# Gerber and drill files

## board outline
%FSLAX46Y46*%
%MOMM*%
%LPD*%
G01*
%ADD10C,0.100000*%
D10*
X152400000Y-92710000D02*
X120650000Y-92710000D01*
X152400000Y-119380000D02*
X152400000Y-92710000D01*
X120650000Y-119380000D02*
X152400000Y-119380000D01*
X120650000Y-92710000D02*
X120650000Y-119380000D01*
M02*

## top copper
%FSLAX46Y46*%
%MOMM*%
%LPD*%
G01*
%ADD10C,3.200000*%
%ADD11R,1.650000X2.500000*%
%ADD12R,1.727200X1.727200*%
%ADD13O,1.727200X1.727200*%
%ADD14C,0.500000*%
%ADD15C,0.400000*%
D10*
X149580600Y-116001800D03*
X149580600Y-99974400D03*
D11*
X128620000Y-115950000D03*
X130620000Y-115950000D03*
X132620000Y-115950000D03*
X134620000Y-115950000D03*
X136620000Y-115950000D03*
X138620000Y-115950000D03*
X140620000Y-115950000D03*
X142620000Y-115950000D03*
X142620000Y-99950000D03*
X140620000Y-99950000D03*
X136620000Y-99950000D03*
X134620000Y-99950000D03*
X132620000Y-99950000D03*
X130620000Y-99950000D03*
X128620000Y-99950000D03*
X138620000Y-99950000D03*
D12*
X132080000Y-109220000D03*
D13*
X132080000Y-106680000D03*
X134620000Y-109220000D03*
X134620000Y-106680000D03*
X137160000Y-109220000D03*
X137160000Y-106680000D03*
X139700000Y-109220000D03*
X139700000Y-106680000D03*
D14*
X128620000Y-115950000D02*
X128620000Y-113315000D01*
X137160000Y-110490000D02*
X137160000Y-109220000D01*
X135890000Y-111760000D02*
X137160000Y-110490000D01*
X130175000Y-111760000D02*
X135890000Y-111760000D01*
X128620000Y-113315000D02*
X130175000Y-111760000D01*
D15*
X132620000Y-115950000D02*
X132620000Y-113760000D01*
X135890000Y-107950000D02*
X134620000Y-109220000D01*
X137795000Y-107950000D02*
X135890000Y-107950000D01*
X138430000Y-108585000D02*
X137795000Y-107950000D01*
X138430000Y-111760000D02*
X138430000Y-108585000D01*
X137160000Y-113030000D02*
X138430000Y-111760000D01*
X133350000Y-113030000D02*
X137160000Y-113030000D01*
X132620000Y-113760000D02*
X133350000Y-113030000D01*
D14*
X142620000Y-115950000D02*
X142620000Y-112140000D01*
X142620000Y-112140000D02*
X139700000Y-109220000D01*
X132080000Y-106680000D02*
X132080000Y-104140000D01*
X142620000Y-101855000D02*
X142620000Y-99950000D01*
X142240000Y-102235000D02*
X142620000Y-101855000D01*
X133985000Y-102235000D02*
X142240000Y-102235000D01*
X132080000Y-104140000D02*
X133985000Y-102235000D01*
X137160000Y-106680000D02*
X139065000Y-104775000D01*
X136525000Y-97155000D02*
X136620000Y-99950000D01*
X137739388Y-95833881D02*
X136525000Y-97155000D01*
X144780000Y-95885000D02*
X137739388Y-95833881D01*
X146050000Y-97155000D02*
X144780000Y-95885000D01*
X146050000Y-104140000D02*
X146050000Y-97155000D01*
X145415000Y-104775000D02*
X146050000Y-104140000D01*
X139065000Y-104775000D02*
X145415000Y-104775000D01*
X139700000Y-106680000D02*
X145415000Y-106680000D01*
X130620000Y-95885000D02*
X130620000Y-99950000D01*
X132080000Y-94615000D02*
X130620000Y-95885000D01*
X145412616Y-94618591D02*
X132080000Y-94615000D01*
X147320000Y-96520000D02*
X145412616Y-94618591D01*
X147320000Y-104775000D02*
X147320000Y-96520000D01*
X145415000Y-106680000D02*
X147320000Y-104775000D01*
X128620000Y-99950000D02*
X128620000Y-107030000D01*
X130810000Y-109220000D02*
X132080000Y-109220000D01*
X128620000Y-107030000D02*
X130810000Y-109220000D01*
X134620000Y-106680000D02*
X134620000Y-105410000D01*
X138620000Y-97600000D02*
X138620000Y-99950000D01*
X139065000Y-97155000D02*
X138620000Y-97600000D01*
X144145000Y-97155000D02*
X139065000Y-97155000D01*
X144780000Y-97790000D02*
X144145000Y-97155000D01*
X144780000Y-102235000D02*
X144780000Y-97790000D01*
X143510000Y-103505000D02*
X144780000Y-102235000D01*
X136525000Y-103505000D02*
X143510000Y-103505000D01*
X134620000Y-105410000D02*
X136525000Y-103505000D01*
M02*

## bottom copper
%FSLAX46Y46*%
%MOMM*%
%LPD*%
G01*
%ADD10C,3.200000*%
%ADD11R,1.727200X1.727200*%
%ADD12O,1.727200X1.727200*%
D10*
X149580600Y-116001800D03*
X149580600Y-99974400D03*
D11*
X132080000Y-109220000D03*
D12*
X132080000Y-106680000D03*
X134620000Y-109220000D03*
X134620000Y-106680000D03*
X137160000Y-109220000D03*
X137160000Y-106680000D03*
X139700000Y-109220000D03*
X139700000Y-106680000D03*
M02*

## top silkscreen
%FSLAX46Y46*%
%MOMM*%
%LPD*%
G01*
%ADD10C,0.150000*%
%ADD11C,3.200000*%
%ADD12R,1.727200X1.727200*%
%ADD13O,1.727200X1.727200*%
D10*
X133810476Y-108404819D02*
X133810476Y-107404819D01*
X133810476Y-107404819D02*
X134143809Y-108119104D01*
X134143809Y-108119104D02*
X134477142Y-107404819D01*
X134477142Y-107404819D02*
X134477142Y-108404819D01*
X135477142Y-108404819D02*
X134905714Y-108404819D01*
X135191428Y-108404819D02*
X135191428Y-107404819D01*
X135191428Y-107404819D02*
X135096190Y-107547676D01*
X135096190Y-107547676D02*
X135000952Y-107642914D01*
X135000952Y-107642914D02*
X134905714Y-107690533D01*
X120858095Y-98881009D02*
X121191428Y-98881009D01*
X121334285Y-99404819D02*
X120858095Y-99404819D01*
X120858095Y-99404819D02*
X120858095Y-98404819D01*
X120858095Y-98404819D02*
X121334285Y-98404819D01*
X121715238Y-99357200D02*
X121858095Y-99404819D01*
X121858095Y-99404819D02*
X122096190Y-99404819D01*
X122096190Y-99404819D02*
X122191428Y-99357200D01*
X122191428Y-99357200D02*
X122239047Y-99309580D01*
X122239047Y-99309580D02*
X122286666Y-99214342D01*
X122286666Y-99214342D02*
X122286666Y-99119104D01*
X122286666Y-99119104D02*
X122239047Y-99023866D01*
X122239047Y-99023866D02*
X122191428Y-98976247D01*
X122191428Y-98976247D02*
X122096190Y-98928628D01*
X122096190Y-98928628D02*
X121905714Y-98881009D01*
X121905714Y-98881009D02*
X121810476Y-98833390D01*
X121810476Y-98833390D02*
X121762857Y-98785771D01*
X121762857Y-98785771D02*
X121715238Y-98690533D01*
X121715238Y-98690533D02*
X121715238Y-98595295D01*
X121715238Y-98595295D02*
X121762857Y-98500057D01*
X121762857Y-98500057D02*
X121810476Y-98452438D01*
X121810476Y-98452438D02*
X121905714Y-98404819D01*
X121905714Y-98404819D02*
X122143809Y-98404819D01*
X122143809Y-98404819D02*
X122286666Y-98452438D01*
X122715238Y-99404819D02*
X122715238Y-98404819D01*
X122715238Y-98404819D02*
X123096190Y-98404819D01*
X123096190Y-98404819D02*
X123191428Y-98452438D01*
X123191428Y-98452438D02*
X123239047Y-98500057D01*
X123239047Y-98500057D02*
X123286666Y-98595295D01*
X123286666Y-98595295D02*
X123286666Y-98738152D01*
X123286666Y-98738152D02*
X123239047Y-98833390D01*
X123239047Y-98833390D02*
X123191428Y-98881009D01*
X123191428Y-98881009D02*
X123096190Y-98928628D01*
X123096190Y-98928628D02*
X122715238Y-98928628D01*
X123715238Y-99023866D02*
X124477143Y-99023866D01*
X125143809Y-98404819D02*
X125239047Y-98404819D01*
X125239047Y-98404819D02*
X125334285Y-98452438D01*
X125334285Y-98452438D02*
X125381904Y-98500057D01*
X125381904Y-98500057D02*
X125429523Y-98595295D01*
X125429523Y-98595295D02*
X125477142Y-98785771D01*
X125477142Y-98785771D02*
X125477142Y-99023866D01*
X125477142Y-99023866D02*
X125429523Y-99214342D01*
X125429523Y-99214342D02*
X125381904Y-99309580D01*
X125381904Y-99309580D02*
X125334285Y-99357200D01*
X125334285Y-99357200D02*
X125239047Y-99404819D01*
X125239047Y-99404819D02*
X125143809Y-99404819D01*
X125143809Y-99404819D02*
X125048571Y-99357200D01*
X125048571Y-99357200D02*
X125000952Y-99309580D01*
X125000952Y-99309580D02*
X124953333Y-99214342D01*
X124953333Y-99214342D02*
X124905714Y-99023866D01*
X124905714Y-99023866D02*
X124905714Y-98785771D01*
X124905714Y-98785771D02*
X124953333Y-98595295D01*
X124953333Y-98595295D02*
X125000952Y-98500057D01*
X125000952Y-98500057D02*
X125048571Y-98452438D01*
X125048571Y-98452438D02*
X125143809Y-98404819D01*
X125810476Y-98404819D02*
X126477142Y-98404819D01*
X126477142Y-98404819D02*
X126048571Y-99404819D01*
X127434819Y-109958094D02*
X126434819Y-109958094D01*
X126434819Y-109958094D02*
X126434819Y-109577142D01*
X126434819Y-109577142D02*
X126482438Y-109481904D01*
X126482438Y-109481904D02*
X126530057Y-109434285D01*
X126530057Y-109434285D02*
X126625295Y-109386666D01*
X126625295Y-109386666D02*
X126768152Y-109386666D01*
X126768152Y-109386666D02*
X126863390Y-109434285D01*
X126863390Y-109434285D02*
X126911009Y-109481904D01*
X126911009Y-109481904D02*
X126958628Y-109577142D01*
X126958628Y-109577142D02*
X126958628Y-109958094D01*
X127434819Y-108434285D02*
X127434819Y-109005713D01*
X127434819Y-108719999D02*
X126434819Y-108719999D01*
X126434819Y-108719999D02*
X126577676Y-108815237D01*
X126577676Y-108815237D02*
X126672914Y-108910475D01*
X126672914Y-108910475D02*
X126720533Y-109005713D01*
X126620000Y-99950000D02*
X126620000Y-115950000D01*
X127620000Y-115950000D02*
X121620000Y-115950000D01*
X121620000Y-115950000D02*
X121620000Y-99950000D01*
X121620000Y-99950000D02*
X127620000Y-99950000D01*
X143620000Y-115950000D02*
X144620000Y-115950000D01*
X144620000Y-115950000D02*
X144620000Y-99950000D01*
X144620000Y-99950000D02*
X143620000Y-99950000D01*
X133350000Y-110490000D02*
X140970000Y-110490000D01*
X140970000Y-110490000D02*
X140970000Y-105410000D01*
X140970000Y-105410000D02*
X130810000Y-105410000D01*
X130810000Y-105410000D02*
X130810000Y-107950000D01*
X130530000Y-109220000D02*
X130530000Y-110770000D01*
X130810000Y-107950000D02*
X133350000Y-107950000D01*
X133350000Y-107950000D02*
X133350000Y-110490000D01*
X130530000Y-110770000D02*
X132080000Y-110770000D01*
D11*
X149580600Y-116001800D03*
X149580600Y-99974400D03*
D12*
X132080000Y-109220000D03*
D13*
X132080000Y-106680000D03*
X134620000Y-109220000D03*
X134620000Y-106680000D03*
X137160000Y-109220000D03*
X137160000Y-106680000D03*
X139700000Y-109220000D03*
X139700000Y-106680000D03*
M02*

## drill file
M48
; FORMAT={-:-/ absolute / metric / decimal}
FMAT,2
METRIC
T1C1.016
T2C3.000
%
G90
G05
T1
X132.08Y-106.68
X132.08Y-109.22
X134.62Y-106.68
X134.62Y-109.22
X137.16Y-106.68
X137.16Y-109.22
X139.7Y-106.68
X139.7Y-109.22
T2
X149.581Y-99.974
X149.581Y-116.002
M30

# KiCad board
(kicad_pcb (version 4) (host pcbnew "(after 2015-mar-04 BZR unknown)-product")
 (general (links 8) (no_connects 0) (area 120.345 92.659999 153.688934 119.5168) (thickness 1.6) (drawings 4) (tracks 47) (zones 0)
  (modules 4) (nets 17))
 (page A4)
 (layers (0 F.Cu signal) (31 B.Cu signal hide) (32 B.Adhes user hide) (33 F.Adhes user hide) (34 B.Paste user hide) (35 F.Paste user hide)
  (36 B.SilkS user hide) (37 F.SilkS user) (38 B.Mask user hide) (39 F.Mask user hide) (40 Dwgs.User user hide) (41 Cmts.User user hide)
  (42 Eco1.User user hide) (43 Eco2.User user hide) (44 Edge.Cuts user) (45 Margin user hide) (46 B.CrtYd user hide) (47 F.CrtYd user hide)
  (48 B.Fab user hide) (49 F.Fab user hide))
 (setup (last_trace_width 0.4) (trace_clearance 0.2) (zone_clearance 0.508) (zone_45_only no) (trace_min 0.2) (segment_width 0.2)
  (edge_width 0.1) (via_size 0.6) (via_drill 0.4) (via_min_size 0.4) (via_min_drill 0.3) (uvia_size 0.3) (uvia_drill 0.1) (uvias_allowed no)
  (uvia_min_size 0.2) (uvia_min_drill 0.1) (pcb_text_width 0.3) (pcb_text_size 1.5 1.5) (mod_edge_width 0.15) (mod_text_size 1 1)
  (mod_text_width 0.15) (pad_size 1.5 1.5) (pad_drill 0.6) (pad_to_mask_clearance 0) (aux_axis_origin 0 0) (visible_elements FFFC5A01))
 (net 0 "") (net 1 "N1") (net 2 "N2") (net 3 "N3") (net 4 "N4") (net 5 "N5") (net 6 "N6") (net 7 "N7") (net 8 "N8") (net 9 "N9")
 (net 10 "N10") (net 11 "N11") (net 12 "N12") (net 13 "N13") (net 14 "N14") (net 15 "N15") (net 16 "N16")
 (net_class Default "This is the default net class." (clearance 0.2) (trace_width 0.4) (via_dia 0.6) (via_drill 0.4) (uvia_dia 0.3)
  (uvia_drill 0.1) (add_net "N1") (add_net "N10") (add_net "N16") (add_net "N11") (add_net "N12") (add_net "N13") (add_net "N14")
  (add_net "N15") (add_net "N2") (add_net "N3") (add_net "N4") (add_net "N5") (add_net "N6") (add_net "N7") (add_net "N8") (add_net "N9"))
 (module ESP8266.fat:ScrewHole (layer F.Cu) (at 149.5806 116.0018)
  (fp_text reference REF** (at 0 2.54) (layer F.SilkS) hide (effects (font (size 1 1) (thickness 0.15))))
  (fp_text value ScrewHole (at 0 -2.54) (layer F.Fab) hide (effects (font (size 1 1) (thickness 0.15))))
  (pad 1 thru_hole circle (at 0 0) (size 3.2 3.2) (drill 3) (layers *.Cu *.Mask F.SilkS)))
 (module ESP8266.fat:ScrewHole (layer F.Cu) (at 149.5806 99.9744)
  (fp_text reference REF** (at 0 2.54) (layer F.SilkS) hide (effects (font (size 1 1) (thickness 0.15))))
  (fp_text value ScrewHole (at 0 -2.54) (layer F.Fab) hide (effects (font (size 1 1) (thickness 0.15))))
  (pad 1 thru_hole circle (at 0 0) (size 3.2 3.2) (drill 3) (layers *.Cu *.Mask F.SilkS)))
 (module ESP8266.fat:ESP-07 (layer F.Cu) (at 134.62 107.95)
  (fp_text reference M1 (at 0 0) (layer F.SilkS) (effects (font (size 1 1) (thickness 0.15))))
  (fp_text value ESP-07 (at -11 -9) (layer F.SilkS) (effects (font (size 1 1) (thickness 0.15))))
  (fp_line (start -8 -8) (end -8 8) (layer F.SilkS) (width 0.15))
  (fp_line (start -7 8) (end -13 8) (layer F.SilkS) (width 0.15))
  (fp_line (start -13 8) (end -13 -8) (layer F.SilkS) (width 0.15))
  (fp_line (start -13 -8) (end -7 -8) (layer F.SilkS) (width 0.15))
  (fp_line (start 9 8) (end 10 8) (layer F.SilkS) (width 0.15))
  (fp_line (start 10 8) (end 10 -8) (layer F.SilkS) (width 0.15))
  (fp_line (start 10 -8) (end 9 -8) (layer F.SilkS) (width 0.15))
  (pad 1 smd rect (at -6 8) (size 1.65 2.5) (layers F.Cu F.Paste F.Mask) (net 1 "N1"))
  (pad 2 smd rect (at -4 8) (size 1.65 2.5) (layers F.Cu F.Paste F.Mask) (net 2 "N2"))
  (pad 3 smd rect (at -2 8) (size 1.65 2.5) (layers F.Cu F.Paste F.Mask) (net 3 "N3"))
  (pad 4 smd rect (at 0 8) (size 1.65 2.5) (layers F.Cu F.Paste F.Mask) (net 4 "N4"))
  (pad 5 smd rect (at 2 8) (size 1.65 2.5) (layers F.Cu F.Paste F.Mask) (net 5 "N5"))
  (pad 6 smd rect (at 4 8) (size 1.65 2.5) (layers F.Cu F.Paste F.Mask) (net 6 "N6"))
  (pad 7 smd rect (at 6 8) (size 1.65 2.5) (layers F.Cu F.Paste F.Mask) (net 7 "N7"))
  (pad 8 smd rect (at 8 8) (size 1.65 2.5) (layers F.Cu F.Paste F.Mask) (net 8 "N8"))
  (pad 9 smd rect (at 8 -8) (size 1.65 2.5) (layers F.Cu F.Paste F.Mask) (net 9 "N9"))
  (pad 10 smd rect (at 6 -8) (size 1.65 2.5) (layers F.Cu F.Paste F.Mask) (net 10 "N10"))
  (pad 12 smd rect (at 2 -8) (size 1.65 2.5) (layers F.Cu F.Paste F.Mask) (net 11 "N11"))
  (pad 13 smd rect (at 0 -8) (size 1.65 2.5) (layers F.Cu F.Paste F.Mask) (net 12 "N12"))
  (pad 14 smd rect (at -2 -8) (size 1.65 2.5) (layers F.Cu F.Paste F.Mask) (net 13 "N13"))
  (pad 15 smd rect (at -4 -8) (size 1.65 2.5) (layers F.Cu F.Paste F.Mask) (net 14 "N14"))
  (pad 16 smd rect (at -6 -8) (size 1.65 2.5) (layers F.Cu F.Paste F.Mask) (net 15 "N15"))
  (pad 11 smd rect (at 4 -8) (size 1.65 2.5) (layers F.Cu F.Paste F.Mask) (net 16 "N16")))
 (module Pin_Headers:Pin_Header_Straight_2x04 (layer F.Cu) (at 132.08 109.22 90)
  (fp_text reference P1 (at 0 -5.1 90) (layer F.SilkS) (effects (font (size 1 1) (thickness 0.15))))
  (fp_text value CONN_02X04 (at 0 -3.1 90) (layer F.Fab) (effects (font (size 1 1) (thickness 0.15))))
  (fp_line (start -1.27 1.27) (end -1.27 8.89) (layer F.SilkS) (width 0.15))
  (fp_line (start -1.27 8.89) (end 3.81 8.89) (layer F.SilkS) (width 0.15))
  (fp_line (start 3.81 8.89) (end 3.81 -1.27) (layer F.SilkS) (width 0.15))
  (fp_line (start 3.81 -1.27) (end 1.27 -1.27) (layer F.SilkS) (width 0.15))
  (fp_line (start 0 -1.55) (end -1.55 -1.55) (layer F.SilkS) (width 0.15))
  (fp_line (start 1.27 -1.27) (end 1.27 1.27) (layer F.SilkS) (width 0.15))
  (fp_line (start 1.27 1.27) (end -1.27 1.27) (layer F.SilkS) (width 0.15))
  (fp_line (start -1.55 -1.55) (end -1.55 0) (layer F.SilkS) (width 0.15))
  (pad 1 thru_hole rect (at 0 0 90) (size 1.7272 1.7272) (drill 1.016) (layers *.Cu *.Mask F.SilkS) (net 15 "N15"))
  (pad 2 thru_hole oval (at 2.54 0 90) (size 1.7272 1.7272) (drill 1.016) (layers *.Cu *.Mask F.SilkS) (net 9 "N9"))
  (pad 3 thru_hole oval (at 0 2.54 90) (size 1.7272 1.7272) (drill 1.016) (layers *.Cu *.Mask F.SilkS) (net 3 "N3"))
  (pad 4 thru_hole oval (at 2.54 2.54 90) (size 1.7272 1.7272) (drill 1.016) (layers *.Cu *.Mask F.SilkS) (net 16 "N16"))
  (pad 5 thru_hole oval (at 0 5.08 90) (size 1.7272 1.7272) (drill 1.016) (layers *.Cu *.Mask F.SilkS) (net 1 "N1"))
  (pad 6 thru_hole oval (at 2.54 5.08 90) (size 1.7272 1.7272) (drill 1.016) (layers *.Cu *.Mask F.SilkS) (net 11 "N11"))
  (pad 7 thru_hole oval (at 0 7.62 90) (size 1.7272 1.7272) (drill 1.016) (layers *.Cu *.Mask F.SilkS) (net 8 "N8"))
  (pad 8 thru_hole oval (at 2.54 7.62 90) (size 1.7272 1.7272) (drill 1.016) (layers *.Cu *.Mask F.SilkS) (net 14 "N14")))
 (gr_line (start 152.4 92.71) (end 120.65 92.71) (angle 90) (layer Edge.Cuts) (width 0.1))
 (gr_line (start 152.4 119.38) (end 152.4 92.71) (angle 90) (layer Edge.Cuts) (width 0.1))
 (gr_line (start 120.65 119.38) (end 152.4 119.38) (angle 90) (layer Edge.Cuts) (width 0.1))
 (gr_line (start 120.65 92.71) (end 120.65 119.38) (angle 90) (layer Edge.Cuts) (width 0.1))
 (segment (start 128.62 115.95) (end 128.62 113.315) (width 0.5) (layer F.Cu) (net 1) (status 400000))
 (segment (start 137.16 110.49) (end 137.16 109.22) (width 0.5) (layer F.Cu) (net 1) (status 800000))
 (segment (start 135.89 111.76) (end 137.16 110.49) (width 0.5) (layer F.Cu) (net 1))
 (segment (start 130.175 111.76) (end 135.89 111.76) (width 0.5) (layer F.Cu) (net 1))
 (segment (start 128.62 113.315) (end 130.175 111.76) (width 0.5) (layer F.Cu) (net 1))
 (segment (start 132.62 115.95) (end 132.62 113.76) (width 0.4) (layer F.Cu) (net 3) (status 400000))
 (segment (start 135.89 107.95) (end 134.62 109.22) (width 0.4) (layer F.Cu) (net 3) (status 800000))
 (segment (start 137.795 107.95) (end 135.89 107.95) (width 0.4) (layer F.Cu) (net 3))
 (segment (start 138.43 108.585) (end 137.795 107.95) (width 0.4) (layer F.Cu) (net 3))
 (segment (start 138.43 111.76) (end 138.43 108.585) (width 0.4) (layer F.Cu) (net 3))
 (segment (start 137.16 113.03) (end 138.43 111.76) (width 0.4) (layer F.Cu) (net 3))
 (segment (start 133.35 113.03) (end 137.16 113.03) (width 0.4) (layer F.Cu) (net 3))
 (segment (start 132.62 113.76) (end 133.35 113.03) (width 0.4) (layer F.Cu) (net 3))
 (segment (start 142.62 115.95) (end 142.62 112.14) (width 0.5) (layer F.Cu) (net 8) (status 400000))
 (segment (start 142.62 112.14) (end 139.7 109.22) (width 0.5) (layer F.Cu) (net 8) (status 800000))
 (segment (start 132.08 106.68) (end 132.08 104.14) (width 0.5) (layer F.Cu) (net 9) (status 400000))
 (segment (start 142.62 101.855) (end 142.62 99.95) (width 0.5) (layer F.Cu) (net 9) (status 800000))
 (segment (start 142.24 102.235) (end 142.62 101.855) (width 0.5) (layer F.Cu) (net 9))
 (segment (start 133.985 102.235) (end 142.24 102.235) (width 0.5) (layer F.Cu) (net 9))
 (segment (start 132.08 104.14) (end 133.985 102.235) (width 0.5) (layer F.Cu) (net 9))
 (segment (start 137.16 106.68) (end 139.065 104.775) (width 0.5) (layer F.Cu) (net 11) (status 400000))
 (segment (start 136.525 97.155) (end 136.62 99.95) (width 0.5) (layer F.Cu) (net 11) (status 800000))
 (segment (start 137.739388 95.833881) (end 136.525 97.155) (width 0.5) (layer F.Cu) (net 11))
 (segment (start 144.78 95.885) (end 137.739388 95.833881) (width 0.5) (layer F.Cu) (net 11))
 (segment (start 146.05 97.155) (end 144.78 95.885) (width 0.5) (layer F.Cu) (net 11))
 (segment (start 146.05 104.14) (end 146.05 97.155) (width 0.5) (layer F.Cu) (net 11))
 (segment (start 145.415 104.775) (end 146.05 104.14) (width 0.5) (layer F.Cu) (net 11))
 (segment (start 139.065 104.775) (end 145.415 104.775) (width 0.5) (layer F.Cu) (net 11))
 (segment (start 139.7 106.68) (end 145.415 106.68) (width 0.5) (layer F.Cu) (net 14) (status 400000))
 (segment (start 130.62 95.885) (end 130.62 99.95) (width 0.5) (layer F.Cu) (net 14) (status 800000))
 (segment (start 132.08 94.615) (end 130.62 95.885) (width 0.5) (layer F.Cu) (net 14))
 (segment (start 145.412616 94.618591) (end 132.08 94.615) (width 0.5) (layer F.Cu) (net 14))
 (segment (start 147.32 96.52) (end 145.412616 94.618591) (width 0.5) (layer F.Cu) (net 14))
 (segment (start 147.32 104.775) (end 147.32 96.52) (width 0.5) (layer F.Cu) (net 14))
 (segment (start 145.415 106.68) (end 147.32 104.775) (width 0.5) (layer F.Cu) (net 14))
 (segment (start 128.62 99.95) (end 128.62 107.03) (width 0.5) (layer F.Cu) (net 15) (status 400000))
 (segment (start 130.81 109.22) (end 132.08 109.22) (width 0.5) (layer F.Cu) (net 15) (status 800000))
 (segment (start 128.62 107.03) (end 130.81 109.22) (width 0.5) (layer F.Cu) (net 15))
 (segment (start 134.62 106.68) (end 134.62 105.41) (width 0.5) (layer F.Cu) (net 16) (status 400000))
 (segment (start 138.62 97.6) (end 138.62 99.95) (width 0.5) (layer F.Cu) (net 16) (status 800000))
 (segment (start 139.065 97.155) (end 138.62 97.6) (width 0.5) (layer F.Cu) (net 16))
 (segment (start 144.145 97.155) (end 139.065 97.155) (width 0.5) (layer F.Cu) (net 16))
 (segment (start 144.78 97.79) (end 144.145 97.155) (width 0.5) (layer F.Cu) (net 16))
 (segment (start 144.78 102.235) (end 144.78 97.79) (width 0.5) (layer F.Cu) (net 16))
 (segment (start 143.51 103.505) (end 144.78 102.235) (width 0.5) (layer F.Cu) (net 16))
 (segment (start 136.525 103.505) (end 143.51 103.505) (width 0.5) (layer F.Cu) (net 16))
 (segment (start 134.62 105.41) (end 136.525 103.505) (width 0.5) (layer F.Cu) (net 16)))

